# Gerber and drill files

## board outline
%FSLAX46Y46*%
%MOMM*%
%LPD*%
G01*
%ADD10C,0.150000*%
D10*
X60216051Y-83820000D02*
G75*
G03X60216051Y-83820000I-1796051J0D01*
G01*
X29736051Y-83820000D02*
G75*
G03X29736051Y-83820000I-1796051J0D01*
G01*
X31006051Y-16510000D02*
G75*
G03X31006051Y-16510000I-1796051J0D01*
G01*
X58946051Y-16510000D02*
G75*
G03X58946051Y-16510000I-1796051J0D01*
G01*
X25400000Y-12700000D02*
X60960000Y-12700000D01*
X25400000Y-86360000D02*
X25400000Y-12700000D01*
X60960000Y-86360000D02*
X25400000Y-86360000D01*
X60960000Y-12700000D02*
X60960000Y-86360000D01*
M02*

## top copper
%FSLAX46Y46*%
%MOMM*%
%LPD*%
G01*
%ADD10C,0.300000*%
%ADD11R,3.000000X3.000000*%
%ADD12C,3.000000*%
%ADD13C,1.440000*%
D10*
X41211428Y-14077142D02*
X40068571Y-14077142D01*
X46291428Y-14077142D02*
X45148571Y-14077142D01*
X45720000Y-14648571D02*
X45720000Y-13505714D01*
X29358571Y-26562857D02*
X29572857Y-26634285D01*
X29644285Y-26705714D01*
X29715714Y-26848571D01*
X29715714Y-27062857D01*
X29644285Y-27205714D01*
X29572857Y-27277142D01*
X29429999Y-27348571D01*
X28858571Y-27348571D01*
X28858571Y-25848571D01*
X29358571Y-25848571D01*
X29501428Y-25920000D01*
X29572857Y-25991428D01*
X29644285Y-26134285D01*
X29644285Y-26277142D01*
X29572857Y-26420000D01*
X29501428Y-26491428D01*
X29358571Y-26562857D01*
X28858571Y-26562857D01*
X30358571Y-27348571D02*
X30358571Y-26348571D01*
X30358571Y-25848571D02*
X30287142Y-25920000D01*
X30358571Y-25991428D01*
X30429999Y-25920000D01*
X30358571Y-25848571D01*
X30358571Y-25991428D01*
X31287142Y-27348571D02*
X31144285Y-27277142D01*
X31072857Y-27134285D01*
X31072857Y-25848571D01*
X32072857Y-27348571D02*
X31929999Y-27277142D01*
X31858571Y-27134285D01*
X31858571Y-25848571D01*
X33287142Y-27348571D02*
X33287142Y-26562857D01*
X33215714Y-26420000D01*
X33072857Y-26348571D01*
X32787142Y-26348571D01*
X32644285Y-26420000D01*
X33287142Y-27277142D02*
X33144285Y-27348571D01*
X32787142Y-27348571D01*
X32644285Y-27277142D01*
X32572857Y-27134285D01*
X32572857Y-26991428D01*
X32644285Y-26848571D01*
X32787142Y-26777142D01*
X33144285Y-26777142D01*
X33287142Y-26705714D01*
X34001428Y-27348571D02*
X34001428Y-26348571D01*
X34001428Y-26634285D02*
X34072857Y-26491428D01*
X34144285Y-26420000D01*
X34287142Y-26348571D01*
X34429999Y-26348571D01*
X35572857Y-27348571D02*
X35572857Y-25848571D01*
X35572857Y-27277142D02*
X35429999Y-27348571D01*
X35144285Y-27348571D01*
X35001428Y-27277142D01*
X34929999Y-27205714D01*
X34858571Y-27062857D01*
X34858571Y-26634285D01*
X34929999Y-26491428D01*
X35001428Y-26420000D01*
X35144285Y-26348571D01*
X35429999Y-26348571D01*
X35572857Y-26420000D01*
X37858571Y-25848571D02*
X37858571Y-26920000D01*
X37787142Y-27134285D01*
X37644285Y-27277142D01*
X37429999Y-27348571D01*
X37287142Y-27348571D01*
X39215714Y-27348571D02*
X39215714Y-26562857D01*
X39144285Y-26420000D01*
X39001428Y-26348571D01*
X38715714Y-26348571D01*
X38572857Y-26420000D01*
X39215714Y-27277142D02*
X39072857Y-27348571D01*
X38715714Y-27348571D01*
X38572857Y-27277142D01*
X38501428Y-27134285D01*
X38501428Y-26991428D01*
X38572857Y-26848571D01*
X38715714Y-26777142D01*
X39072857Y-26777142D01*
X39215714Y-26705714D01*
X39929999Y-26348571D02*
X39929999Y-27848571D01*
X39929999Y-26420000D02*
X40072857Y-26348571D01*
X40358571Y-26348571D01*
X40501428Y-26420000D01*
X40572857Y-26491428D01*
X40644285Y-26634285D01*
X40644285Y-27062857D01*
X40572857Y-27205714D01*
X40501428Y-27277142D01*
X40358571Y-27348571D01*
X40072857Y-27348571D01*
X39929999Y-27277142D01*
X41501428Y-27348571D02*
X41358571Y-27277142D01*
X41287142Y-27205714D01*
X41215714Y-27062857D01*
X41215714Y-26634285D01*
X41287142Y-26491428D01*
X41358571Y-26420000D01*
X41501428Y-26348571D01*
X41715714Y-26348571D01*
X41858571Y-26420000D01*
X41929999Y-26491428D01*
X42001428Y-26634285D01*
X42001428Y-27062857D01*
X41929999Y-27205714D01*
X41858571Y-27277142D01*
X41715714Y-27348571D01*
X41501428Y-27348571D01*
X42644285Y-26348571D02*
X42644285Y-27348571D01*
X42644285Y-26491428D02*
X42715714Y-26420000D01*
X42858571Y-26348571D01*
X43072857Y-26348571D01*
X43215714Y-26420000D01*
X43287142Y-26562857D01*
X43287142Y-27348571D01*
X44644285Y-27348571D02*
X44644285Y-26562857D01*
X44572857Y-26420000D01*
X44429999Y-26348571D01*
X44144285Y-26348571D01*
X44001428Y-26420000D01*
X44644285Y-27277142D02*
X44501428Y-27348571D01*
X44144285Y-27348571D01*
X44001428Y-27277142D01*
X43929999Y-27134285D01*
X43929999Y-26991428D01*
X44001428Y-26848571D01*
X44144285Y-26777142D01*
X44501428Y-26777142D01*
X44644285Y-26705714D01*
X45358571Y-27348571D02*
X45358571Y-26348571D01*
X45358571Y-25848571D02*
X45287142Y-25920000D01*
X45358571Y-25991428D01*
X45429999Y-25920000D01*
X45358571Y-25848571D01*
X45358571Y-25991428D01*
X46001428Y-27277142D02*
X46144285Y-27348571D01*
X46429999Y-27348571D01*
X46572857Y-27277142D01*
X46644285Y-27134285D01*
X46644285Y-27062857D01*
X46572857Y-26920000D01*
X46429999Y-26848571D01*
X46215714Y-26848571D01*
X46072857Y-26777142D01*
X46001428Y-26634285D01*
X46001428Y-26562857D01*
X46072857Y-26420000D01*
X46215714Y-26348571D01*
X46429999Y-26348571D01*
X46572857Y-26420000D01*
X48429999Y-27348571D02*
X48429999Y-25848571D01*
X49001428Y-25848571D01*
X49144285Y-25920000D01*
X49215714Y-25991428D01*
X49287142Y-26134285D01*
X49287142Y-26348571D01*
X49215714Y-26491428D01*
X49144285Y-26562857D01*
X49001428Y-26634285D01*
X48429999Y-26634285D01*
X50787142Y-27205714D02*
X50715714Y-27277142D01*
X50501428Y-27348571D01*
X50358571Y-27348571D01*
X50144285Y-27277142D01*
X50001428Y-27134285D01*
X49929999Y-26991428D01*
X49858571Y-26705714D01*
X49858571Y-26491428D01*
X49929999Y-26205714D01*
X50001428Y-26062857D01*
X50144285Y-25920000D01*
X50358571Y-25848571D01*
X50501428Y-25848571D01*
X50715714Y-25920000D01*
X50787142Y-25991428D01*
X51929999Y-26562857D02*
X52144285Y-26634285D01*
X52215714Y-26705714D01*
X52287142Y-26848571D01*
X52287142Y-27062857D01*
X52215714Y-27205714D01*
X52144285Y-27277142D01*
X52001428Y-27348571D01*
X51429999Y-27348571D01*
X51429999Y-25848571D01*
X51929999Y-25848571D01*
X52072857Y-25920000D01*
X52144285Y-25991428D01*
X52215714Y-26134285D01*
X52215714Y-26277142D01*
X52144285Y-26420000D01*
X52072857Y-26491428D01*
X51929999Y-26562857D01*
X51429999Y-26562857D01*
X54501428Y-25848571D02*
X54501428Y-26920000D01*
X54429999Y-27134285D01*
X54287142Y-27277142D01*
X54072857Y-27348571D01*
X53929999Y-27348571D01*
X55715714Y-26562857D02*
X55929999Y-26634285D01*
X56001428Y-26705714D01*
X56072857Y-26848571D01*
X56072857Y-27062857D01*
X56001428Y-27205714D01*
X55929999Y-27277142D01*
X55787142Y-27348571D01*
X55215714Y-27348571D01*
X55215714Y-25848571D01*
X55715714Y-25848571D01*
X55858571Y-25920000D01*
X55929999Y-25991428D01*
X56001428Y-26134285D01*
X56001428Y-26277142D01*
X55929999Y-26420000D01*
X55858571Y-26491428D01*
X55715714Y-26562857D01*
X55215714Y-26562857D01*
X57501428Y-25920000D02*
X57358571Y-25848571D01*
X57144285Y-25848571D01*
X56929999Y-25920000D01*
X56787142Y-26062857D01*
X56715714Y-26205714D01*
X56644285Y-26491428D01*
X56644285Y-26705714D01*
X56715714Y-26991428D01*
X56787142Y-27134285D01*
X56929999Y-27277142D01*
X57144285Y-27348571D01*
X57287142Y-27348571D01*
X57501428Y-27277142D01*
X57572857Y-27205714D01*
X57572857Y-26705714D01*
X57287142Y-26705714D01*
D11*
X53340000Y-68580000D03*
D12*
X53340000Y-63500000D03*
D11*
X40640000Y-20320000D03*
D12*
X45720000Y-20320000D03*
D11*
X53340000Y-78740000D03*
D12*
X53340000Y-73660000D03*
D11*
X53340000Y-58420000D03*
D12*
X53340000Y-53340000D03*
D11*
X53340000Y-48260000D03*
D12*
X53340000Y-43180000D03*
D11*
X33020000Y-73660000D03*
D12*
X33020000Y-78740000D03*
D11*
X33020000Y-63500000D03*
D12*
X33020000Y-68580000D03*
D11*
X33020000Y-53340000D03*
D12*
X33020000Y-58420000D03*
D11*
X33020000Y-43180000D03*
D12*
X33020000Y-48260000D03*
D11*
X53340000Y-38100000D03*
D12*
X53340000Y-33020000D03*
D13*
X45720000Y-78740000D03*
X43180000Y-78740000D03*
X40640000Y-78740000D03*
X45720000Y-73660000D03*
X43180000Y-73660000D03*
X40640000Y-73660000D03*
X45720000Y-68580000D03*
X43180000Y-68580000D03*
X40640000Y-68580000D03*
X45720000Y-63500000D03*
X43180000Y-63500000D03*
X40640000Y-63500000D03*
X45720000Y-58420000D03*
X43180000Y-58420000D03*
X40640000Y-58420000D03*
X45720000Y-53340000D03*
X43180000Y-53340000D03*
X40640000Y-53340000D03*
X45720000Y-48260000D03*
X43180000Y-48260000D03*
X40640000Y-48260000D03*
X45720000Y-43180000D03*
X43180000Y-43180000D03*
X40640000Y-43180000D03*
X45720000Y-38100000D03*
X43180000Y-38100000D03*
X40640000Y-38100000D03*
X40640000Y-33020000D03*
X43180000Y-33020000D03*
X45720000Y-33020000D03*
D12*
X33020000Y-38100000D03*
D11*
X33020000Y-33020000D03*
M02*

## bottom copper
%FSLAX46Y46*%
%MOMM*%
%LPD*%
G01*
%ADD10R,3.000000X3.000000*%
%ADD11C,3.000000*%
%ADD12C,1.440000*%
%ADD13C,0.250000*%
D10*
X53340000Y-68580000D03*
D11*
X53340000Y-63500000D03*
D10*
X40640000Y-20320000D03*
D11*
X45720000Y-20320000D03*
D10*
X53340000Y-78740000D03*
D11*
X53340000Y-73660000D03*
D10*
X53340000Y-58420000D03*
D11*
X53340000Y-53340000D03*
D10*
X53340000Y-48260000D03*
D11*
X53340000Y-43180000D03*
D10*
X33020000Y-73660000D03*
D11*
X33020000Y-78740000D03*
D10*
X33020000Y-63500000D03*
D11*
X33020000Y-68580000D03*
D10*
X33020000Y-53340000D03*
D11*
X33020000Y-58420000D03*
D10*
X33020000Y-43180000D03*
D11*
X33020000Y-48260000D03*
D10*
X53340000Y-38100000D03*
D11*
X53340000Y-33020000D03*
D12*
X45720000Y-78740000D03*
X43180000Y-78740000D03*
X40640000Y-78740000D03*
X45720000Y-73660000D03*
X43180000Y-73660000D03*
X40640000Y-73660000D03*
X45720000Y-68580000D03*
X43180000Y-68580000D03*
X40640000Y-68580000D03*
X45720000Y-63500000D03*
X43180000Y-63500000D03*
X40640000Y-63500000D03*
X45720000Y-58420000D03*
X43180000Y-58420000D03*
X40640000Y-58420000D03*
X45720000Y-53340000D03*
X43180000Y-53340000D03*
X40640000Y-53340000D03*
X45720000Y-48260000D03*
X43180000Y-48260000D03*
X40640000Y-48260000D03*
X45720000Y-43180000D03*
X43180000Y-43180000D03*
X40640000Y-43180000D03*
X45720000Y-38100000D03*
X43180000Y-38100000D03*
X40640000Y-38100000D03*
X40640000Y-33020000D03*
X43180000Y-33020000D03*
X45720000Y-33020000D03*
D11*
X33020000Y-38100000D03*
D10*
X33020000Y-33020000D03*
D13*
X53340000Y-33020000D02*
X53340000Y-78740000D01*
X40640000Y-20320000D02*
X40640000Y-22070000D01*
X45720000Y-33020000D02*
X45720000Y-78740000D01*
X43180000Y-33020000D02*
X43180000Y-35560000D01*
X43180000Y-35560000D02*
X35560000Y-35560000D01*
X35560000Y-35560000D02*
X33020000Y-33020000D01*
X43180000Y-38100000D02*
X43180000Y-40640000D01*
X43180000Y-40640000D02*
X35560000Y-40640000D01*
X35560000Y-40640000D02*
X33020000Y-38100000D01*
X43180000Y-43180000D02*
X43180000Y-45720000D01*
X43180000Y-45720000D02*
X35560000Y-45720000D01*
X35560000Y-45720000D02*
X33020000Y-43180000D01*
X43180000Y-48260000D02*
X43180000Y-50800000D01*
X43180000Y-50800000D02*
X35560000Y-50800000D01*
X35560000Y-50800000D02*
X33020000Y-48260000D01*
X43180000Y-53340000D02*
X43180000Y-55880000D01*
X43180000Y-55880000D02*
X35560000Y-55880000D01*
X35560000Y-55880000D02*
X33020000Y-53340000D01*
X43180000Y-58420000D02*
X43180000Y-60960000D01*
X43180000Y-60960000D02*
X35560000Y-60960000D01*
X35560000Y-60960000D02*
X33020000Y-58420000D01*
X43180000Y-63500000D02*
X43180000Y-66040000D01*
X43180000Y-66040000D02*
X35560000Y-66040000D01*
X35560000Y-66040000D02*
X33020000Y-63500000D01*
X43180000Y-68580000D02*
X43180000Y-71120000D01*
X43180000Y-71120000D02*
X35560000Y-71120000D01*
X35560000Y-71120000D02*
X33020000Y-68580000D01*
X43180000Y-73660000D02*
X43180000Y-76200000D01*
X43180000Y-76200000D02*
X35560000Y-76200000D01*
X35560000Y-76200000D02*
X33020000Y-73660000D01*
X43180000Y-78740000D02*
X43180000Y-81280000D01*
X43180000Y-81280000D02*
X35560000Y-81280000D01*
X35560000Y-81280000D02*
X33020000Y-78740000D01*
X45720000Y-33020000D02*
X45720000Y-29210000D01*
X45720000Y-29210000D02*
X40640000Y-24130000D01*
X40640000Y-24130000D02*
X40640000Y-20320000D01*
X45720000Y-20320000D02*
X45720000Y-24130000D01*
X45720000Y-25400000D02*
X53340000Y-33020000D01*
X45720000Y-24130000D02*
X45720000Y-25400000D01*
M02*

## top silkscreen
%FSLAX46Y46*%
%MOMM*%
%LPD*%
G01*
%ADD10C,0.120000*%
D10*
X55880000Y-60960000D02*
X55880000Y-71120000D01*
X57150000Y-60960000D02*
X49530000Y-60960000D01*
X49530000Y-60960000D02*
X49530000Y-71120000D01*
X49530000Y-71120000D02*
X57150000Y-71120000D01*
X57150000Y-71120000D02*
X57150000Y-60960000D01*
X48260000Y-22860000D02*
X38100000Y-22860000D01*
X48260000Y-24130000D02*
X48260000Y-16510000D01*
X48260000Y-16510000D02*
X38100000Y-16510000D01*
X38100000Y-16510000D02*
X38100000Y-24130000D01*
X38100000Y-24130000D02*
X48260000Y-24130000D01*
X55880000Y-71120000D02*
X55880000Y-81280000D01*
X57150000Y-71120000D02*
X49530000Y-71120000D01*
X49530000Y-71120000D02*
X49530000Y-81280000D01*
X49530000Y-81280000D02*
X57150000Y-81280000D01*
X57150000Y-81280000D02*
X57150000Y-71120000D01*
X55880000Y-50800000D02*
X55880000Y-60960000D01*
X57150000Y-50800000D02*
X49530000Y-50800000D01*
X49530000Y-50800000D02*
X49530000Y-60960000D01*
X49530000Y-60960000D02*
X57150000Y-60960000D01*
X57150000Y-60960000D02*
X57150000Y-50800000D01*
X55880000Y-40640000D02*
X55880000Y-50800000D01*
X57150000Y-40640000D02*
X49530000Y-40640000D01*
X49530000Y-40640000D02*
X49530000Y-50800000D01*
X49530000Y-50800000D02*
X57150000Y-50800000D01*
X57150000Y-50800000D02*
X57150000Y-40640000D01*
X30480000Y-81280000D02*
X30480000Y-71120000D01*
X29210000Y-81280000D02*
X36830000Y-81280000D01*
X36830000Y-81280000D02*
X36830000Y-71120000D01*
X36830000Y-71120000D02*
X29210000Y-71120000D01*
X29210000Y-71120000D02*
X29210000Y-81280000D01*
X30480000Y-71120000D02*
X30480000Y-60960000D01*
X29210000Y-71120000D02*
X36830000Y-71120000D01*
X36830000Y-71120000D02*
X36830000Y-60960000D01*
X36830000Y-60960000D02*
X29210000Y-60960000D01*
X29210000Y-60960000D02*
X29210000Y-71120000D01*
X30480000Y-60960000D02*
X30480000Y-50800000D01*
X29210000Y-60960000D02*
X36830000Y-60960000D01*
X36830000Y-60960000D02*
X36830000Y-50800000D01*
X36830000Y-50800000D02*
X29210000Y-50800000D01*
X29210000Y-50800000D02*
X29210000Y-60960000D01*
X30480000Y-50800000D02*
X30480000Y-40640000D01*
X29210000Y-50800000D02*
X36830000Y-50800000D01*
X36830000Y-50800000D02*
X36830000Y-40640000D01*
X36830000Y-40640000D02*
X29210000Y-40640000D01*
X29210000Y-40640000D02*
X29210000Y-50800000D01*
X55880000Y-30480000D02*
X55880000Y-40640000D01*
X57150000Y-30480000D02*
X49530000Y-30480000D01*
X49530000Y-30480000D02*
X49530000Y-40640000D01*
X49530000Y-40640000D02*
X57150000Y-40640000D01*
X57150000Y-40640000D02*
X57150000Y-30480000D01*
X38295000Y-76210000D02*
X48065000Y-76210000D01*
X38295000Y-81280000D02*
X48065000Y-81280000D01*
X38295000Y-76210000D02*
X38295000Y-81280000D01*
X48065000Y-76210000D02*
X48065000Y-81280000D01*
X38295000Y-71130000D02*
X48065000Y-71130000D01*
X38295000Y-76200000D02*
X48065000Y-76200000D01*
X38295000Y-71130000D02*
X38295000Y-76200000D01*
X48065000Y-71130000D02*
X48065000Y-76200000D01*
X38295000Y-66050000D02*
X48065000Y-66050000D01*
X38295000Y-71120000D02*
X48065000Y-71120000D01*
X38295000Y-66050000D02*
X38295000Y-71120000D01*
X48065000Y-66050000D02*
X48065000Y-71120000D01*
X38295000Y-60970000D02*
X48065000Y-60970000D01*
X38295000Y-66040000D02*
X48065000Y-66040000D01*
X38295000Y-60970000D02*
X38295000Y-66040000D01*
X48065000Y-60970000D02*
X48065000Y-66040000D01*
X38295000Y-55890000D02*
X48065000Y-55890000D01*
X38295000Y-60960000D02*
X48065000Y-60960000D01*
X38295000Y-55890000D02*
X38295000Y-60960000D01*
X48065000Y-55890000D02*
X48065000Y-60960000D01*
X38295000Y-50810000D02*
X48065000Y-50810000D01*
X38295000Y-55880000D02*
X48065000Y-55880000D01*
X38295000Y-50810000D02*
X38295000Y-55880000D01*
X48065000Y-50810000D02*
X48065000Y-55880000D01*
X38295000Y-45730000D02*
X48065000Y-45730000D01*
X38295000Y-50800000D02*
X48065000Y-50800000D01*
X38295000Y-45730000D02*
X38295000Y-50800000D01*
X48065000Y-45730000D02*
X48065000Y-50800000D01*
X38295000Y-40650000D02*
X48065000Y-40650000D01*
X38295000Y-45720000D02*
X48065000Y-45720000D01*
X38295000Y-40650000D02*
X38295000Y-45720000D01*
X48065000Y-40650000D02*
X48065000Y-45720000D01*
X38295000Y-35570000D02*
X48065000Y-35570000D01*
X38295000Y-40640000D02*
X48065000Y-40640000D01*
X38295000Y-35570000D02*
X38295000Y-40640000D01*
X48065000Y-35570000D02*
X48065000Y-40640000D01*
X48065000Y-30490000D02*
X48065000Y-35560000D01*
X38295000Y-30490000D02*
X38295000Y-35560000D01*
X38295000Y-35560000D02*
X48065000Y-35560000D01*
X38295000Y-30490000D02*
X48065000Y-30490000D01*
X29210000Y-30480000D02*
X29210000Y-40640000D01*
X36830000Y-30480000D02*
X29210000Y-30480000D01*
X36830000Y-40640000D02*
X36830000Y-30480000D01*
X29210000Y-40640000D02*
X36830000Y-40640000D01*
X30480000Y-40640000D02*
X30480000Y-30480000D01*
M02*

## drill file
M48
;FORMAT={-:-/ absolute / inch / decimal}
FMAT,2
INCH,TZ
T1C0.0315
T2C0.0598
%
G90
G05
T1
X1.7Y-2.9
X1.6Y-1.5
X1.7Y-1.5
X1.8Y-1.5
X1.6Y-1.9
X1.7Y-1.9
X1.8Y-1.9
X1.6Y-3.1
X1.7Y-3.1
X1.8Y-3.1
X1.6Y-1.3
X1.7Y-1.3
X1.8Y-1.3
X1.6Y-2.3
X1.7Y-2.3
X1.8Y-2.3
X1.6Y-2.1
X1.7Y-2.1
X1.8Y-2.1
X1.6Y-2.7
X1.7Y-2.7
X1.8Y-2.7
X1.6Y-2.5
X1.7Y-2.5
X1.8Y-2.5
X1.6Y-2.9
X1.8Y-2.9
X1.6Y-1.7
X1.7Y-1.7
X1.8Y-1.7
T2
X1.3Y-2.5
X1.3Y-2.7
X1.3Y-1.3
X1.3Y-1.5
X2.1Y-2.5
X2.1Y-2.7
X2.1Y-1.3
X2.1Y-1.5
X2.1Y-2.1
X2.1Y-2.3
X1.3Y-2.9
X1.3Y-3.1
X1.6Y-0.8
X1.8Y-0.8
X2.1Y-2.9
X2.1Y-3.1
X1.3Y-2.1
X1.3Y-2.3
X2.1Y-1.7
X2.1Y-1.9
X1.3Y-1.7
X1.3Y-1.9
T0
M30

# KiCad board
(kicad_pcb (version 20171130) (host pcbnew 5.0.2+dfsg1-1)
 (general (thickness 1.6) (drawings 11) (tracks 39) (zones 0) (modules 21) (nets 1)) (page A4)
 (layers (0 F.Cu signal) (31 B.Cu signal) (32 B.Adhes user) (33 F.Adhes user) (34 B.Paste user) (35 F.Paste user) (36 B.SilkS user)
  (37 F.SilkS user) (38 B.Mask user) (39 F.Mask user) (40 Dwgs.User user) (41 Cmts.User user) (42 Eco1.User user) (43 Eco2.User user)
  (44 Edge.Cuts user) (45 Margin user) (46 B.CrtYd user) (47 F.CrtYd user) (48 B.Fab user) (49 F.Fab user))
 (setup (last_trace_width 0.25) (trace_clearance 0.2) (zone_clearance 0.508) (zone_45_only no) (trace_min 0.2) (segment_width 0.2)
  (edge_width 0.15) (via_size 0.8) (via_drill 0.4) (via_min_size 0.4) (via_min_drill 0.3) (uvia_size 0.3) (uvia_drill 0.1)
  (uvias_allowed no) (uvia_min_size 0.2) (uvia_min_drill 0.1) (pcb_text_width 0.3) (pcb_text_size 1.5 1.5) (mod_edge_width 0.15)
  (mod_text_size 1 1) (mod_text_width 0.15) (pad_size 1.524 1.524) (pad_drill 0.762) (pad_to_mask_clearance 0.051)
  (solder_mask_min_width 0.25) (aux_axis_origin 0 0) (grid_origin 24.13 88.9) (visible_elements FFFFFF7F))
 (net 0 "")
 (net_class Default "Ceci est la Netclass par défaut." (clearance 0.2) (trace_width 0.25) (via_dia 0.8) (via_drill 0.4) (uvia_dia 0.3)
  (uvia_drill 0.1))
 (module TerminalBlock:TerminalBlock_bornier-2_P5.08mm (layer F.Cu) (at 53.34 68.58 90)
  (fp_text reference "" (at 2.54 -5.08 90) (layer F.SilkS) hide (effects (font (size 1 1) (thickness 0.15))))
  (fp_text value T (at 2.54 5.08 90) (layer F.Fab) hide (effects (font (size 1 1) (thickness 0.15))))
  (fp_line (start 7.62 2.54) (end -2.54 2.54) (layer F.SilkS) (width 0.12))
  (fp_line (start 7.62 3.81) (end 7.62 -3.81) (layer F.SilkS) (width 0.12))
  (fp_line (start 7.62 -3.81) (end -2.54 -3.81) (layer F.SilkS) (width 0.12))
  (fp_line (start -2.54 -3.81) (end -2.54 3.81) (layer F.SilkS) (width 0.12))
  (fp_line (start -2.54 3.81) (end 7.62 3.81) (layer F.SilkS) (width 0.12))
  (pad 1 thru_hole rect (at 0 0 90) (size 3 3) (drill 1.52) (layers *.Cu *.Mask))
  (pad 2 thru_hole circle (at 5.08 0 90) (size 3 3) (drill 1.52) (layers *.Cu *.Mask)))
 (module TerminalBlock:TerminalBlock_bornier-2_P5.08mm (layer F.Cu) (at 40.64 20.32)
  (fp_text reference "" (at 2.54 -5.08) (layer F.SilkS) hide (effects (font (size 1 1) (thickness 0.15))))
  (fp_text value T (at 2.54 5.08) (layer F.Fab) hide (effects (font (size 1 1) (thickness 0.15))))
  (fp_line (start 7.62 2.54) (end -2.54 2.54) (layer F.SilkS) (width 0.12))
  (fp_line (start 7.62 3.81) (end 7.62 -3.81) (layer F.SilkS) (width 0.12))
  (fp_line (start 7.62 -3.81) (end -2.54 -3.81) (layer F.SilkS) (width 0.12))
  (fp_line (start -2.54 -3.81) (end -2.54 3.81) (layer F.SilkS) (width 0.12))
  (fp_line (start -2.54 3.81) (end 7.62 3.81) (layer F.SilkS) (width 0.12))
  (pad 1 thru_hole rect (at 0 0) (size 3 3) (drill 1.52) (layers *.Cu *.Mask))
  (pad 2 thru_hole circle (at 5.08 0) (size 3 3) (drill 1.52) (layers *.Cu *.Mask)))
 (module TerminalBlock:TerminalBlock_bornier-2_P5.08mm (layer F.Cu) (at 53.34 78.74 90)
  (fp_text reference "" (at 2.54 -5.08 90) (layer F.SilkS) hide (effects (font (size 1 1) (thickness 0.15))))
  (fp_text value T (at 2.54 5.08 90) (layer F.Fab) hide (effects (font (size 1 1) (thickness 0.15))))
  (fp_line (start 7.62 2.54) (end -2.54 2.54) (layer F.SilkS) (width 0.12))
  (fp_line (start 7.62 3.81) (end 7.62 -3.81) (layer F.SilkS) (width 0.12))
  (fp_line (start 7.62 -3.81) (end -2.54 -3.81) (layer F.SilkS) (width 0.12))
  (fp_line (start -2.54 -3.81) (end -2.54 3.81) (layer F.SilkS) (width 0.12))
  (fp_line (start -2.54 3.81) (end 7.62 3.81) (layer F.SilkS) (width 0.12))
  (pad 1 thru_hole rect (at 0 0 90) (size 3 3) (drill 1.52) (layers *.Cu *.Mask))
  (pad 2 thru_hole circle (at 5.08 0 90) (size 3 3) (drill 1.52) (layers *.Cu *.Mask)))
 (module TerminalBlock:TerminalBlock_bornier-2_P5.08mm (layer F.Cu) (at 53.34 58.42 90)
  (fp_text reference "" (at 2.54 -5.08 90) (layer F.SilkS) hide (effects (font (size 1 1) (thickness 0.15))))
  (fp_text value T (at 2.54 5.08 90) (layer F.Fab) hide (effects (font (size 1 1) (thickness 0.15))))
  (fp_line (start 7.62 2.54) (end -2.54 2.54) (layer F.SilkS) (width 0.12))
  (fp_line (start 7.62 3.81) (end 7.62 -3.81) (layer F.SilkS) (width 0.12))
  (fp_line (start 7.62 -3.81) (end -2.54 -3.81) (layer F.SilkS) (width 0.12))
  (fp_line (start -2.54 -3.81) (end -2.54 3.81) (layer F.SilkS) (width 0.12))
  (fp_line (start -2.54 3.81) (end 7.62 3.81) (layer F.SilkS) (width 0.12))
  (pad 1 thru_hole rect (at 0 0 90) (size 3 3) (drill 1.52) (layers *.Cu *.Mask))
  (pad 2 thru_hole circle (at 5.08 0 90) (size 3 3) (drill 1.52) (layers *.Cu *.Mask)))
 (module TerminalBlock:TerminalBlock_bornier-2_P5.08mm (layer F.Cu) (at 53.34 48.26 90)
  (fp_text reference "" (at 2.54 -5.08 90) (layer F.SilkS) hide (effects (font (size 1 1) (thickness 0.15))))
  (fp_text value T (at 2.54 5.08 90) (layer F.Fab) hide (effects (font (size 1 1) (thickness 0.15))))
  (fp_line (start 7.62 2.54) (end -2.54 2.54) (layer F.SilkS) (width 0.12))
  (fp_line (start 7.62 3.81) (end 7.62 -3.81) (layer F.SilkS) (width 0.12))
  (fp_line (start 7.62 -3.81) (end -2.54 -3.81) (layer F.SilkS) (width 0.12))
  (fp_line (start -2.54 -3.81) (end -2.54 3.81) (layer F.SilkS) (width 0.12))
  (fp_line (start -2.54 3.81) (end 7.62 3.81) (layer F.SilkS) (width 0.12))
  (pad 1 thru_hole rect (at 0 0 90) (size 3 3) (drill 1.52) (layers *.Cu *.Mask))
  (pad 2 thru_hole circle (at 5.08 0 90) (size 3 3) (drill 1.52) (layers *.Cu *.Mask)))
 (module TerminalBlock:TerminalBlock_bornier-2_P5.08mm (layer F.Cu) (at 33.02 73.66 270)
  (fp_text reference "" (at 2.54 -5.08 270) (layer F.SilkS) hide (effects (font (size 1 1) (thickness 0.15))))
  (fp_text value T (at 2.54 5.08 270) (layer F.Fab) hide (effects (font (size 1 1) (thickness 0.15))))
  (fp_line (start 7.62 2.54) (end -2.54 2.54) (layer F.SilkS) (width 0.12))
  (fp_line (start 7.62 3.81) (end 7.62 -3.81) (layer F.SilkS) (width 0.12))
  (fp_line (start 7.62 -3.81) (end -2.54 -3.81) (layer F.SilkS) (width 0.12))
  (fp_line (start -2.54 -3.81) (end -2.54 3.81) (layer F.SilkS) (width 0.12))
  (fp_line (start -2.54 3.81) (end 7.62 3.81) (layer F.SilkS) (width 0.12))
  (pad 1 thru_hole rect (at 0 0 270) (size 3 3) (drill 1.52) (layers *.Cu *.Mask))
  (pad 2 thru_hole circle (at 5.08 0 270) (size 3 3) (drill 1.52) (layers *.Cu *.Mask)))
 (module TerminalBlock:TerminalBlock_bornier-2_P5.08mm (layer F.Cu) (at 33.02 63.5 270)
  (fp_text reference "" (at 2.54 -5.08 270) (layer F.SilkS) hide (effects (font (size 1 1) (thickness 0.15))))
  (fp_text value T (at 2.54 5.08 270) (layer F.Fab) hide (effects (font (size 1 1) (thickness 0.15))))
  (fp_line (start 7.62 2.54) (end -2.54 2.54) (layer F.SilkS) (width 0.12))
  (fp_line (start 7.62 3.81) (end 7.62 -3.81) (layer F.SilkS) (width 0.12))
  (fp_line (start 7.62 -3.81) (end -2.54 -3.81) (layer F.SilkS) (width 0.12))
  (fp_line (start -2.54 -3.81) (end -2.54 3.81) (layer F.SilkS) (width 0.12))
  (fp_line (start -2.54 3.81) (end 7.62 3.81) (layer F.SilkS) (width 0.12))
  (pad 1 thru_hole rect (at 0 0 270) (size 3 3) (drill 1.52) (layers *.Cu *.Mask))
  (pad 2 thru_hole circle (at 5.08 0 270) (size 3 3) (drill 1.52) (layers *.Cu *.Mask)))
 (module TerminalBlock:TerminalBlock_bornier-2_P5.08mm (layer F.Cu) (at 33.02 53.34 270)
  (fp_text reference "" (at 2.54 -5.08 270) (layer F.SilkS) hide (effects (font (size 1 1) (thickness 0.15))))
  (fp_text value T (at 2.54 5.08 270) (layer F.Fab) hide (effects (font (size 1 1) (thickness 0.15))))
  (fp_line (start 7.62 2.54) (end -2.54 2.54) (layer F.SilkS) (width 0.12))
  (fp_line (start 7.62 3.81) (end 7.62 -3.81) (layer F.SilkS) (width 0.12))
  (fp_line (start 7.62 -3.81) (end -2.54 -3.81) (layer F.SilkS) (width 0.12))
  (fp_line (start -2.54 -3.81) (end -2.54 3.81) (layer F.SilkS) (width 0.12))
  (fp_line (start -2.54 3.81) (end 7.62 3.81) (layer F.SilkS) (width 0.12))
  (pad 1 thru_hole rect (at 0 0 270) (size 3 3) (drill 1.52) (layers *.Cu *.Mask))
  (pad 2 thru_hole circle (at 5.08 0 270) (size 3 3) (drill 1.52) (layers *.Cu *.Mask)))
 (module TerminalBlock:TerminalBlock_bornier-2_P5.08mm (layer F.Cu) (at 33.02 43.18 270)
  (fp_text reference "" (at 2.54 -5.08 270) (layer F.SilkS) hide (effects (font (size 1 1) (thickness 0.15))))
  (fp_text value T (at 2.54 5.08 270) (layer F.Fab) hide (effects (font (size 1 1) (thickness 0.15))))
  (fp_line (start 7.62 2.54) (end -2.54 2.54) (layer F.SilkS) (width 0.12))
  (fp_line (start 7.62 3.81) (end 7.62 -3.81) (layer F.SilkS) (width 0.12))
  (fp_line (start 7.62 -3.81) (end -2.54 -3.81) (layer F.SilkS) (width 0.12))
  (fp_line (start -2.54 -3.81) (end -2.54 3.81) (layer F.SilkS) (width 0.12))
  (fp_line (start -2.54 3.81) (end 7.62 3.81) (layer F.SilkS) (width 0.12))
  (pad 1 thru_hole rect (at 0 0 270) (size 3 3) (drill 1.52) (layers *.Cu *.Mask))
  (pad 2 thru_hole circle (at 5.08 0 270) (size 3 3) (drill 1.52) (layers *.Cu *.Mask)))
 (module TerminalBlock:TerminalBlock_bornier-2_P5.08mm (layer F.Cu) (at 53.34 38.1 90)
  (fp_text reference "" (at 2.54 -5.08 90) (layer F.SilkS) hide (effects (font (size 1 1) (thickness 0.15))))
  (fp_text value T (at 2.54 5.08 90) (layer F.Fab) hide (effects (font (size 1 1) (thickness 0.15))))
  (fp_line (start 7.62 2.54) (end -2.54 2.54) (layer F.SilkS) (width 0.12))
  (fp_line (start 7.62 3.81) (end 7.62 -3.81) (layer F.SilkS) (width 0.12))
  (fp_line (start 7.62 -3.81) (end -2.54 -3.81) (layer F.SilkS) (width 0.12))
  (fp_line (start -2.54 -3.81) (end -2.54 3.81) (layer F.SilkS) (width 0.12))
  (fp_line (start -2.54 3.81) (end 7.62 3.81) (layer F.SilkS) (width 0.12))
  (pad 1 thru_hole rect (at 0 0 90) (size 3 3) (drill 1.52) (layers *.Cu *.Mask))
  (pad 2 thru_hole circle (at 5.08 0 90) (size 3 3) (drill 1.52) (layers *.Cu *.Mask)))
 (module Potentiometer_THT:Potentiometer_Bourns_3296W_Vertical (layer F.Cu) (at 45.72 78.74)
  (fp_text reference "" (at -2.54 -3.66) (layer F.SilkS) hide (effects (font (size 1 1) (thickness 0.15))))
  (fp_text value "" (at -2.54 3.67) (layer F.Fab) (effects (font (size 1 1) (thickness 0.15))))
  (fp_line (start -7.425 -2.53) (end 2.345 -2.53) (layer F.SilkS) (width 0.12))
  (fp_line (start -7.425 2.54) (end 2.345 2.54) (layer F.SilkS) (width 0.12))
  (fp_line (start -7.425 -2.53) (end -7.425 2.54) (layer F.SilkS) (width 0.12))
  (fp_line (start 2.345 -2.53) (end 2.345 2.54) (layer F.SilkS) (width 0.12))
  (pad 1 thru_hole circle (at 0 0) (size 1.44 1.44) (drill 0.8) (layers *.Cu *.Mask))
  (pad 2 thru_hole circle (at -2.54 0) (size 1.44 1.44) (drill 0.8) (layers *.Cu *.Mask))
  (pad 3 thru_hole circle (at -5.08 0) (size 1.44 1.44) (drill 0.8) (layers *.Cu *.Mask)))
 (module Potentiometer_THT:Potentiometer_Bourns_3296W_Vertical (layer F.Cu) (at 45.72 73.66)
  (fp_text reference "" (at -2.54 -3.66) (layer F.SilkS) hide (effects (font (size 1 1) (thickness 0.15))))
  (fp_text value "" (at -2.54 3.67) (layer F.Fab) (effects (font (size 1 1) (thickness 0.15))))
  (fp_line (start -7.425 -2.53) (end 2.345 -2.53) (layer F.SilkS) (width 0.12))
  (fp_line (start -7.425 2.54) (end 2.345 2.54) (layer F.SilkS) (width 0.12))
  (fp_line (start -7.425 -2.53) (end -7.425 2.54) (layer F.SilkS) (width 0.12))
  (fp_line (start 2.345 -2.53) (end 2.345 2.54) (layer F.SilkS) (width 0.12))
  (pad 1 thru_hole circle (at 0 0) (size 1.44 1.44) (drill 0.8) (layers *.Cu *.Mask))
  (pad 2 thru_hole circle (at -2.54 0) (size 1.44 1.44) (drill 0.8) (layers *.Cu *.Mask))
  (pad 3 thru_hole circle (at -5.08 0) (size 1.44 1.44) (drill 0.8) (layers *.Cu *.Mask)))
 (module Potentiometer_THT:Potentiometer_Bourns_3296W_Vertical (layer F.Cu) (at 45.72 68.58)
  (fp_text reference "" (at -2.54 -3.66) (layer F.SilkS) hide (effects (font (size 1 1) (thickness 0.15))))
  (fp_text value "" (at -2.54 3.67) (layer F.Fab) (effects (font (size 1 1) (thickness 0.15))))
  (fp_line (start -7.425 -2.53) (end 2.345 -2.53) (layer F.SilkS) (width 0.12))
  (fp_line (start -7.425 2.54) (end 2.345 2.54) (layer F.SilkS) (width 0.12))
  (fp_line (start -7.425 -2.53) (end -7.425 2.54) (layer F.SilkS) (width 0.12))
  (fp_line (start 2.345 -2.53) (end 2.345 2.54) (layer F.SilkS) (width 0.12))
  (pad 1 thru_hole circle (at 0 0) (size 1.44 1.44) (drill 0.8) (layers *.Cu *.Mask))
  (pad 2 thru_hole circle (at -2.54 0) (size 1.44 1.44) (drill 0.8) (layers *.Cu *.Mask))
  (pad 3 thru_hole circle (at -5.08 0) (size 1.44 1.44) (drill 0.8) (layers *.Cu *.Mask)))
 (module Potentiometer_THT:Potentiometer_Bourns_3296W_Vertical (layer F.Cu) (at 45.72 63.5)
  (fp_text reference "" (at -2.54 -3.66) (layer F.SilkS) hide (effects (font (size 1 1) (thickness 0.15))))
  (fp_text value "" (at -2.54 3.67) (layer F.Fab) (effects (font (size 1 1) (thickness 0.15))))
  (fp_line (start -7.425 -2.53) (end 2.345 -2.53) (layer F.SilkS) (width 0.12))
  (fp_line (start -7.425 2.54) (end 2.345 2.54) (layer F.SilkS) (width 0.12))
  (fp_line (start -7.425 -2.53) (end -7.425 2.54) (layer F.SilkS) (width 0.12))
  (fp_line (start 2.345 -2.53) (end 2.345 2.54) (layer F.SilkS) (width 0.12))
  (pad 1 thru_hole circle (at 0 0) (size 1.44 1.44) (drill 0.8) (layers *.Cu *.Mask))
  (pad 2 thru_hole circle (at -2.54 0) (size 1.44 1.44) (drill 0.8) (layers *.Cu *.Mask))
  (pad 3 thru_hole circle (at -5.08 0) (size 1.44 1.44) (drill 0.8) (layers *.Cu *.Mask)))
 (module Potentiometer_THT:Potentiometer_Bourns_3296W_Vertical (layer F.Cu) (at 45.72 58.42)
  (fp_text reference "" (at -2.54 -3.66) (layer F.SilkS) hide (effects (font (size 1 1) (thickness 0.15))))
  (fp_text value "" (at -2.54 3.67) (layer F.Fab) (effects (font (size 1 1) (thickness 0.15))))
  (fp_line (start -7.425 -2.53) (end 2.345 -2.53) (layer F.SilkS) (width 0.12))
  (fp_line (start -7.425 2.54) (end 2.345 2.54) (layer F.SilkS) (width 0.12))
  (fp_line (start -7.425 -2.53) (end -7.425 2.54) (layer F.SilkS) (width 0.12))
  (fp_line (start 2.345 -2.53) (end 2.345 2.54) (layer F.SilkS) (width 0.12))
  (pad 1 thru_hole circle (at 0 0) (size 1.44 1.44) (drill 0.8) (layers *.Cu *.Mask))
  (pad 2 thru_hole circle (at -2.54 0) (size 1.44 1.44) (drill 0.8) (layers *.Cu *.Mask))
  (pad 3 thru_hole circle (at -5.08 0) (size 1.44 1.44) (drill 0.8) (layers *.Cu *.Mask)))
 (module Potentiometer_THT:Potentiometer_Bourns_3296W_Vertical (layer F.Cu) (at 45.72 53.34)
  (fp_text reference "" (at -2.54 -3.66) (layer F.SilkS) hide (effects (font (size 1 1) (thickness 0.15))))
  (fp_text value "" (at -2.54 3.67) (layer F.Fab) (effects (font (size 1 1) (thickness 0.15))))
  (fp_line (start -7.425 -2.53) (end 2.345 -2.53) (layer F.SilkS) (width 0.12))
  (fp_line (start -7.425 2.54) (end 2.345 2.54) (layer F.SilkS) (width 0.12))
  (fp_line (start -7.425 -2.53) (end -7.425 2.54) (layer F.SilkS) (width 0.12))
  (fp_line (start 2.345 -2.53) (end 2.345 2.54) (layer F.SilkS) (width 0.12))
  (pad 1 thru_hole circle (at 0 0) (size 1.44 1.44) (drill 0.8) (layers *.Cu *.Mask))
  (pad 2 thru_hole circle (at -2.54 0) (size 1.44 1.44) (drill 0.8) (layers *.Cu *.Mask))
  (pad 3 thru_hole circle (at -5.08 0) (size 1.44 1.44) (drill 0.8) (layers *.Cu *.Mask)))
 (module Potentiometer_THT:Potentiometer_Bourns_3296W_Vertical (layer F.Cu) (at 45.72 48.26)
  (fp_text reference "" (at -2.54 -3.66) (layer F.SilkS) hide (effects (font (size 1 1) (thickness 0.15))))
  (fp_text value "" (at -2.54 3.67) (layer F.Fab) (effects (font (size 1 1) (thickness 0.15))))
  (fp_line (start -7.425 -2.53) (end 2.345 -2.53) (layer F.SilkS) (width 0.12))
  (fp_line (start -7.425 2.54) (end 2.345 2.54) (layer F.SilkS) (width 0.12))
  (fp_line (start -7.425 -2.53) (end -7.425 2.54) (layer F.SilkS) (width 0.12))
  (fp_line (start 2.345 -2.53) (end 2.345 2.54) (layer F.SilkS) (width 0.12))
  (pad 1 thru_hole circle (at 0 0) (size 1.44 1.44) (drill 0.8) (layers *.Cu *.Mask))
  (pad 2 thru_hole circle (at -2.54 0) (size 1.44 1.44) (drill 0.8) (layers *.Cu *.Mask))
  (pad 3 thru_hole circle (at -5.08 0) (size 1.44 1.44) (drill 0.8) (layers *.Cu *.Mask)))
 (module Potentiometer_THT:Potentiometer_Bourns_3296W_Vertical (layer F.Cu) (at 45.72 43.18)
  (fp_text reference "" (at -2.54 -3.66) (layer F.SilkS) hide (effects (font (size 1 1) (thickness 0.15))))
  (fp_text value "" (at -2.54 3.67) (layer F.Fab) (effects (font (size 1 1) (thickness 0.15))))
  (fp_line (start -7.425 -2.53) (end 2.345 -2.53) (layer F.SilkS) (width 0.12))
  (fp_line (start -7.425 2.54) (end 2.345 2.54) (layer F.SilkS) (width 0.12))
  (fp_line (start -7.425 -2.53) (end -7.425 2.54) (layer F.SilkS) (width 0.12))
  (fp_line (start 2.345 -2.53) (end 2.345 2.54) (layer F.SilkS) (width 0.12))
  (pad 1 thru_hole circle (at 0 0) (size 1.44 1.44) (drill 0.8) (layers *.Cu *.Mask))
  (pad 2 thru_hole circle (at -2.54 0) (size 1.44 1.44) (drill 0.8) (layers *.Cu *.Mask))
  (pad 3 thru_hole circle (at -5.08 0) (size 1.44 1.44) (drill 0.8) (layers *.Cu *.Mask)))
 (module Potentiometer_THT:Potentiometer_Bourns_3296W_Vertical (layer F.Cu) (at 45.72 38.1)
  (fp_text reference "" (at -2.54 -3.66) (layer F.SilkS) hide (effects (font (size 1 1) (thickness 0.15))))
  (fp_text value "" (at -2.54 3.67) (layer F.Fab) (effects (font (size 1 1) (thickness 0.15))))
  (fp_line (start -7.425 -2.53) (end 2.345 -2.53) (layer F.SilkS) (width 0.12))
  (fp_line (start -7.425 2.54) (end 2.345 2.54) (layer F.SilkS) (width 0.12))
  (fp_line (start -7.425 -2.53) (end -7.425 2.54) (layer F.SilkS) (width 0.12))
  (fp_line (start 2.345 -2.53) (end 2.345 2.54) (layer F.SilkS) (width 0.12))
  (pad 1 thru_hole circle (at 0 0) (size 1.44 1.44) (drill 0.8) (layers *.Cu *.Mask))
  (pad 2 thru_hole circle (at -2.54 0) (size 1.44 1.44) (drill 0.8) (layers *.Cu *.Mask))
  (pad 3 thru_hole circle (at -5.08 0) (size 1.44 1.44) (drill 0.8) (layers *.Cu *.Mask)))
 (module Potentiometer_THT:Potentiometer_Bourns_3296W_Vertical (layer F.Cu) (at 45.72 33.02)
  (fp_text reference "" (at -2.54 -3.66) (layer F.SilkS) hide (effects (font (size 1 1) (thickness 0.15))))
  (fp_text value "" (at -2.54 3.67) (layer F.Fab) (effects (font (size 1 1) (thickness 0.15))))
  (fp_line (start 2.345 -2.53) (end 2.345 2.54) (layer F.SilkS) (width 0.12))
  (fp_line (start -7.425 -2.53) (end -7.425 2.54) (layer F.SilkS) (width 0.12))
  (fp_line (start -7.425 2.54) (end 2.345 2.54) (layer F.SilkS) (width 0.12))
  (fp_line (start -7.425 -2.53) (end 2.345 -2.53) (layer F.SilkS) (width 0.12))
  (pad 3 thru_hole circle (at -5.08 0) (size 1.44 1.44) (drill 0.8) (layers *.Cu *.Mask))
  (pad 2 thru_hole circle (at -2.54 0) (size 1.44 1.44) (drill 0.8) (layers *.Cu *.Mask))
  (pad 1 thru_hole circle (at 0 0) (size 1.44 1.44) (drill 0.8) (layers *.Cu *.Mask)))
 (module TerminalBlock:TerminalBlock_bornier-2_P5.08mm (layer F.Cu) (at 33.02 33.02 270)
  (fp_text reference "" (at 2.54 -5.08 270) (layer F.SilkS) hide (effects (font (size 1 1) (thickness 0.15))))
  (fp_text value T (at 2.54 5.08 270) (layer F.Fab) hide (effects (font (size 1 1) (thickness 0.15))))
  (fp_line (start -2.54 3.81) (end 7.62 3.81) (layer F.SilkS) (width 0.12))
  (fp_line (start -2.54 -3.81) (end -2.54 3.81) (layer F.SilkS) (width 0.12))
  (fp_line (start 7.62 -3.81) (end -2.54 -3.81) (layer F.SilkS) (width 0.12))
  (fp_line (start 7.62 3.81) (end 7.62 -3.81) (layer F.SilkS) (width 0.12))
  (fp_line (start 7.62 2.54) (end -2.54 2.54) (layer F.SilkS) (width 0.12))
  (pad 2 thru_hole circle (at 5.08 0 270) (size 3 3) (drill 1.52) (layers *.Cu *.Mask))
  (pad 1 thru_hole rect (at 0 0 270) (size 3 3) (drill 1.52) (layers *.Cu *.Mask)))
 (gr_circle (center 58.42 83.82) (end 59.69 85.09) (layer Edge.Cuts) (width 0.15))
 (gr_circle (center 27.94 83.82) (end 29.21 85.09) (layer Edge.Cuts) (width 0.15))
 (gr_circle (center 29.21 16.51) (end 30.48 17.78) (layer Edge.Cuts) (width 0.15))
 (gr_circle (center 57.15 16.51) (end 58.42 17.78) (layer Edge.Cuts) (width 0.15))
 (gr_line (start 25.4 12.7) (end 60.96 12.7) (layer Edge.Cuts) (width 0.15))
 (gr_line (start 25.4 86.36) (end 25.4 12.7) (layer Edge.Cuts) (width 0.15))
 (gr_line (start 60.96 86.36) (end 25.4 86.36) (layer Edge.Cuts) (width 0.15))
 (gr_line (start 60.96 12.7) (end 60.96 86.36) (layer Edge.Cuts) (width 0.15))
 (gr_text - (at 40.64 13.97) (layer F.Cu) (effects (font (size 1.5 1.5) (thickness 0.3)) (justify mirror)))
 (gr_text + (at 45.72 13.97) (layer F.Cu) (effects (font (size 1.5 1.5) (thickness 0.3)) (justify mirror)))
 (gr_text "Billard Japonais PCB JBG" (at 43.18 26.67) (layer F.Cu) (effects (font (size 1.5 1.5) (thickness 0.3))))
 (segment (start 53.34 33.02) (end 53.34 78.74) (width 0.25) (layer B.Cu) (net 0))
 (segment (start 40.64 20.32) (end 40.64 22.07) (width 0.25) (layer B.Cu) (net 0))
 (segment (start 45.72 33.02) (end 45.72 78.74) (width 0.25) (layer B.Cu) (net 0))
 (segment (start 43.18 33.02) (end 43.18 35.56) (width 0.25) (layer B.Cu) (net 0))
 (segment (start 43.18 35.56) (end 35.56 35.56) (width 0.25) (layer B.Cu) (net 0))
 (segment (start 35.56 35.56) (end 33.02 33.02) (width 0.25) (layer B.Cu) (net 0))
 (segment (start 43.18 38.1) (end 43.18 40.64) (width 0.25) (layer B.Cu) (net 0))
 (segment (start 43.18 40.64) (end 35.56 40.64) (width 0.25) (layer B.Cu) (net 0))
 (segment (start 35.56 40.64) (end 33.02 38.1) (width 0.25) (layer B.Cu) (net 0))
 (segment (start 43.18 43.18) (end 43.18 45.72) (width 0.25) (layer B.Cu) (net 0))
 (segment (start 43.18 45.72) (end 35.56 45.72) (width 0.25) (layer B.Cu) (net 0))
 (segment (start 35.56 45.72) (end 33.02 43.18) (width 0.25) (layer B.Cu) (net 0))
 (segment (start 43.18 48.26) (end 43.18 50.8) (width 0.25) (layer B.Cu) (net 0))
 (segment (start 43.18 50.8) (end 35.56 50.8) (width 0.25) (layer B.Cu) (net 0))
 (segment (start 35.56 50.8) (end 33.02 48.26) (width 0.25) (layer B.Cu) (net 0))
 (segment (start 43.18 53.34) (end 43.18 55.88) (width 0.25) (layer B.Cu) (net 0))
 (segment (start 43.18 55.88) (end 35.56 55.88) (width 0.25) (layer B.Cu) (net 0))
 (segment (start 35.56 55.88) (end 33.02 53.34) (width 0.25) (layer B.Cu) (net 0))
 (segment (start 43.18 58.42) (end 43.18 60.96) (width 0.25) (layer B.Cu) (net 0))
 (segment (start 43.18 60.96) (end 35.56 60.96) (width 0.25) (layer B.Cu) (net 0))
 (segment (start 35.56 60.96) (end 33.02 58.42) (width 0.25) (layer B.Cu) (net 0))
 (segment (start 43.18 63.5) (end 43.18 66.04) (width 0.25) (layer B.Cu) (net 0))
 (segment (start 43.18 66.04) (end 35.56 66.04) (width 0.25) (layer B.Cu) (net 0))
 (segment (start 35.56 66.04) (end 33.02 63.5) (width 0.25) (layer B.Cu) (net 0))
 (segment (start 43.18 68.58) (end 43.18 71.12) (width 0.25) (layer B.Cu) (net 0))
 (segment (start 43.18 71.12) (end 35.56 71.12) (width 0.25) (layer B.Cu) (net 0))
 (segment (start 35.56 71.12) (end 33.02 68.58) (width 0.25) (layer B.Cu) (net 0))
 (segment (start 43.18 73.66) (end 43.18 76.2) (width 0.25) (layer B.Cu) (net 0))
 (segment (start 43.18 76.2) (end 35.56 76.2) (width 0.25) (layer B.Cu) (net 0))
 (segment (start 35.56 76.2) (end 33.02 73.66) (width 0.25) (layer B.Cu) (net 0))
 (segment (start 43.18 78.74) (end 43.18 81.28) (width 0.25) (layer B.Cu) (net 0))
 (segment (start 43.18 81.28) (end 35.56 81.28) (width 0.25) (layer B.Cu) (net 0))
 (segment (start 35.56 81.28) (end 33.02 78.74) (width 0.25) (layer B.Cu) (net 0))
 (segment (start 45.72 33.02) (end 45.72 29.21) (width 0.25) (layer B.Cu) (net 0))
 (segment (start 45.72 29.21) (end 40.64 24.13) (width 0.25) (layer B.Cu) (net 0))
 (segment (start 40.64 24.13) (end 40.64 20.32) (width 0.25) (layer B.Cu) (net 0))
 (segment (start 45.72 20.32) (end 45.72 24.13) (width 0.25) (layer B.Cu) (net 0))
 (segment (start 45.72 25.4) (end 53.34 33.02) (width 0.25) (layer B.Cu) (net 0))
 (segment (start 45.72 24.13) (end 45.72 25.4) (width 0.25) (layer B.Cu) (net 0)))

